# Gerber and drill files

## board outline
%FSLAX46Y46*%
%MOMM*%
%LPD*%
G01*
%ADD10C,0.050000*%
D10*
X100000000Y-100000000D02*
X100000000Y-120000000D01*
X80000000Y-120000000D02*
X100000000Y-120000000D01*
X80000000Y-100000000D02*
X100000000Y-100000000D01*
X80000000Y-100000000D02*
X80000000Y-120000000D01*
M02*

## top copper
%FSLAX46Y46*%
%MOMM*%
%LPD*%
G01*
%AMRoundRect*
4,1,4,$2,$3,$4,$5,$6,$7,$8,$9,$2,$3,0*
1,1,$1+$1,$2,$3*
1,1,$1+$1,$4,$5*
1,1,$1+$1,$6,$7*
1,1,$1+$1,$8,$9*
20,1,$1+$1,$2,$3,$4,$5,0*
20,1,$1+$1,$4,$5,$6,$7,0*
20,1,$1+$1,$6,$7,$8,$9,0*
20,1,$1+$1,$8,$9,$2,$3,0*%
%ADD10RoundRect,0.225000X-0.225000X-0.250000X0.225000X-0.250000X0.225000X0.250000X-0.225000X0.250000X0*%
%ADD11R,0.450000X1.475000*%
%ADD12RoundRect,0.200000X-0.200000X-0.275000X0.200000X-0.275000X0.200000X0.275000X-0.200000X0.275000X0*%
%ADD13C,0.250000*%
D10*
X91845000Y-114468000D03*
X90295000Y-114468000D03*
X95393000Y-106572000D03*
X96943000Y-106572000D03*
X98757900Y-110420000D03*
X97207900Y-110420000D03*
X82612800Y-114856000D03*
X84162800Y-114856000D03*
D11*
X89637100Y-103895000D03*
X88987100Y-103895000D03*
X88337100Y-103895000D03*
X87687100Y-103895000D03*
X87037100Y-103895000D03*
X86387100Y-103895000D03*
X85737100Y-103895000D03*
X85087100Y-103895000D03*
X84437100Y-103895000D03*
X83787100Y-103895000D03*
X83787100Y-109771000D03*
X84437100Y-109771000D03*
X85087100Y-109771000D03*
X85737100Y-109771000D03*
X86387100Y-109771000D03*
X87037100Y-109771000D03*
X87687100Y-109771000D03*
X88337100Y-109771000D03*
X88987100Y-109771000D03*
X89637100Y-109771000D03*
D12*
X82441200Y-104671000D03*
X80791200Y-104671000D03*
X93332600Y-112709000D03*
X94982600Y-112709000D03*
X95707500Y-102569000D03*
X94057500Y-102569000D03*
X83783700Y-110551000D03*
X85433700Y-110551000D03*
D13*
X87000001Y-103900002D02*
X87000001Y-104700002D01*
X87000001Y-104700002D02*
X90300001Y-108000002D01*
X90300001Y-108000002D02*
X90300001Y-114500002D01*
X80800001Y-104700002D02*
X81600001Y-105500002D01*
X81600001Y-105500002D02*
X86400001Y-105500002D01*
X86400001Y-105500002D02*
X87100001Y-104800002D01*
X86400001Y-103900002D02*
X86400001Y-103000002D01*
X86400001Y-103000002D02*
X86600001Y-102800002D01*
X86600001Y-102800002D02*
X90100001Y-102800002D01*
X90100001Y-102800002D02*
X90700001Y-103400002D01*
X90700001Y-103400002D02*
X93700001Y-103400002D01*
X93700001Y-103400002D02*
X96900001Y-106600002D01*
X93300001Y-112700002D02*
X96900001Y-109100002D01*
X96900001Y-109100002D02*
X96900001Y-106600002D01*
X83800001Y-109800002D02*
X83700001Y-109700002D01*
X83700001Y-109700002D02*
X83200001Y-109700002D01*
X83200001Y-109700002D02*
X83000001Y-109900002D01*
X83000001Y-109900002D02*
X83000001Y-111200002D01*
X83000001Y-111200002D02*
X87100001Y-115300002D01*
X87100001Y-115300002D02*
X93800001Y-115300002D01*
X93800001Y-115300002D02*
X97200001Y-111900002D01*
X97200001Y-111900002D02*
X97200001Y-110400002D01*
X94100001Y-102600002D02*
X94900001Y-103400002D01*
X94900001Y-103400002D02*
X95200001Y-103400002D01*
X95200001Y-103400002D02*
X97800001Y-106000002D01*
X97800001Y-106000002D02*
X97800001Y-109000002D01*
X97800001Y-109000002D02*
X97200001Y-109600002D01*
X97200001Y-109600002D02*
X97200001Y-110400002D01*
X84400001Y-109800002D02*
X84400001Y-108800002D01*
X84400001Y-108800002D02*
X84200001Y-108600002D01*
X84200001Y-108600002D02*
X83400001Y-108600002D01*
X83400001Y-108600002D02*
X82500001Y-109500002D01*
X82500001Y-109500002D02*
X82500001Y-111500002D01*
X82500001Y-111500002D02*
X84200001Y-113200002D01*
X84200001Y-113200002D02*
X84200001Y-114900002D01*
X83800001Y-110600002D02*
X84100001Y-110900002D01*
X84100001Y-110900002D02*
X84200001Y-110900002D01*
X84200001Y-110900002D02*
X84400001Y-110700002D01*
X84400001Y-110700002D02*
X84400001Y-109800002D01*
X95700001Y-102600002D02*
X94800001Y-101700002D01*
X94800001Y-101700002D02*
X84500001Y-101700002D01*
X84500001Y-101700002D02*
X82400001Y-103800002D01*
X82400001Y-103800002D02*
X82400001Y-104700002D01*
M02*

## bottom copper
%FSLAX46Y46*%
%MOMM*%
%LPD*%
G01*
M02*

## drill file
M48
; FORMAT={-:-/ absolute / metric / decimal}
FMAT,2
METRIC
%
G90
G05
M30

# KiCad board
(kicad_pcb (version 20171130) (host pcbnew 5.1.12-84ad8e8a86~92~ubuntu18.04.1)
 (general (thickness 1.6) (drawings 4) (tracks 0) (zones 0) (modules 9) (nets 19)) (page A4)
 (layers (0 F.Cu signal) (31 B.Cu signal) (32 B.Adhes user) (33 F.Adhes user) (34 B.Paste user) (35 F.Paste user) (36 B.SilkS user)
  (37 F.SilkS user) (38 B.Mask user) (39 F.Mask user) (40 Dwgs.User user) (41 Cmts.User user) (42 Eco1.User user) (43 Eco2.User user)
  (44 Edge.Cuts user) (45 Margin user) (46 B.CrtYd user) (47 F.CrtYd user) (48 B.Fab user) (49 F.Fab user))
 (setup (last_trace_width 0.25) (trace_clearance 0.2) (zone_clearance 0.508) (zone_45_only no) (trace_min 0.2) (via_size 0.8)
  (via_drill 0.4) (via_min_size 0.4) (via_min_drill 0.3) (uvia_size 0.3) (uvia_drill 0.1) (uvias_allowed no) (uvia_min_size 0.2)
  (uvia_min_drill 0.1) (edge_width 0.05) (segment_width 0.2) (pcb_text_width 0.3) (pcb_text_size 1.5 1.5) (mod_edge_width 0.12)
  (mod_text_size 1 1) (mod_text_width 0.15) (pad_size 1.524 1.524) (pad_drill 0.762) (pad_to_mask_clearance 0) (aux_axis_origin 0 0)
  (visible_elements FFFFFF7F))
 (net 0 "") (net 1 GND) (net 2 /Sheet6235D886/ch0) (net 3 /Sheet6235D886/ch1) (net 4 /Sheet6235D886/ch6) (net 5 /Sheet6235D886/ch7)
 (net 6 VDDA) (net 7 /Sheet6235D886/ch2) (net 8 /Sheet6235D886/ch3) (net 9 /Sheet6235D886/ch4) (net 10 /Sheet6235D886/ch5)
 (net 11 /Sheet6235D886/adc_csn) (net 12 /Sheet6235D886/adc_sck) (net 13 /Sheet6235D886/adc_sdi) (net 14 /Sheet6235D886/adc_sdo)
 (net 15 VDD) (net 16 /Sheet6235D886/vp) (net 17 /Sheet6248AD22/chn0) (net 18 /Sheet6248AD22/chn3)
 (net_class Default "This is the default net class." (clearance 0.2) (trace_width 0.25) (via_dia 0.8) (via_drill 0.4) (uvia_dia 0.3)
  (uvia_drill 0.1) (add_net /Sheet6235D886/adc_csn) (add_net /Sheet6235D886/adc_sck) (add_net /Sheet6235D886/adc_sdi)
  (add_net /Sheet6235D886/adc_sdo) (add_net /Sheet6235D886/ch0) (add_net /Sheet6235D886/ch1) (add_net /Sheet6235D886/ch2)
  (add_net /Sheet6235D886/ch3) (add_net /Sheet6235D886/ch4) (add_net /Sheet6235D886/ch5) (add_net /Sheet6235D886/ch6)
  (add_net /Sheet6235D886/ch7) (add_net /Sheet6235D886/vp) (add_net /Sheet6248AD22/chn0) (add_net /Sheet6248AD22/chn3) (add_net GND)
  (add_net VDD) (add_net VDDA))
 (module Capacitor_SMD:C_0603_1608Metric (layer F.Cu) (at 91.070000 114.468000)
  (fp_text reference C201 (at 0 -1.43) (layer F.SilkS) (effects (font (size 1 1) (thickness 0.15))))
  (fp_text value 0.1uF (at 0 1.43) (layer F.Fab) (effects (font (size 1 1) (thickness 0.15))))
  (pad 2 smd roundrect (at 0.775 0) (size 0.9 0.95) (layers F.Cu F.Mask F.Paste) (roundrect_rratio 0.25) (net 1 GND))
  (pad 1 smd roundrect (at -0.775 0) (size 0.9 0.95) (layers F.Cu F.Mask F.Paste) (roundrect_rratio 0.25) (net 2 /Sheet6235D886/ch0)))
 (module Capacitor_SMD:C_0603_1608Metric (layer F.Cu) (at 96.168000 106.572000)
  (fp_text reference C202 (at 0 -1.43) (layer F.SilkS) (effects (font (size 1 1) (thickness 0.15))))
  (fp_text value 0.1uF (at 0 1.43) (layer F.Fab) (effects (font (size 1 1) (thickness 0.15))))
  (pad 1 smd roundrect (at -0.775 0) (size 0.9 0.95) (layers F.Cu F.Mask F.Paste) (roundrect_rratio 0.25) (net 1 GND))
  (pad 2 smd roundrect (at 0.775 0) (size 0.9 0.95) (layers F.Cu F.Mask F.Paste) (roundrect_rratio 0.25) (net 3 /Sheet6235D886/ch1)))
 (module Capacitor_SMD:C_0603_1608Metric (layer F.Cu) (at 97.982900 110.420000)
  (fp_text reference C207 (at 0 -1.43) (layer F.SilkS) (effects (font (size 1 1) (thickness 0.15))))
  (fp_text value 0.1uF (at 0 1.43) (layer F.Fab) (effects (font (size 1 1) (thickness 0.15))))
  (pad 2 smd roundrect (at 0.775 0) (size 0.9 0.95) (layers F.Cu F.Mask F.Paste) (roundrect_rratio 0.25) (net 1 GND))
  (pad 1 smd roundrect (at -0.775 0) (size 0.9 0.95) (layers F.Cu F.Mask F.Paste) (roundrect_rratio 0.25) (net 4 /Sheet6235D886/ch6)))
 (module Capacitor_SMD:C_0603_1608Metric (layer F.Cu) (at 83.387800 114.856000)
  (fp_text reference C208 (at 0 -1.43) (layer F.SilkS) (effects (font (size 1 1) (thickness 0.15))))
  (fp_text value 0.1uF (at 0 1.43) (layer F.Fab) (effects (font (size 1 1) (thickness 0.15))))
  (pad 1 smd roundrect (at -0.775 0) (size 0.9 0.95) (layers F.Cu F.Mask F.Paste) (roundrect_rratio 0.25) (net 1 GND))
  (pad 2 smd roundrect (at 0.775 0) (size 0.9 0.95) (layers F.Cu F.Mask F.Paste) (roundrect_rratio 0.25) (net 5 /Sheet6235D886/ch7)))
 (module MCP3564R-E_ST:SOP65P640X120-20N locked (layer F.Cu) (at 86.712100 106.833000 270.000000)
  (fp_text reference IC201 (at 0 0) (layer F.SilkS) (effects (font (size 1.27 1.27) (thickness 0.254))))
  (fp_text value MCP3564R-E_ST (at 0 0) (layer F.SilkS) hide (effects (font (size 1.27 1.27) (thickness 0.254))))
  (pad 1 smd rect (at -2.938 -2.925) (size 0.45 1.475) (layers F.Cu F.Mask F.Paste) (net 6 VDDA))
  (pad 2 smd rect (at -2.938 -2.275) (size 0.45 1.475) (layers F.Cu F.Mask F.Paste) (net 1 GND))
  (pad 3 smd rect (at -2.938 -1.625) (size 0.45 1.475) (layers F.Cu F.Mask F.Paste) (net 1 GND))
  (pad 4 smd rect (at -2.938 -0.975) (size 0.45 1.475) (layers F.Cu F.Mask F.Paste))
  (pad 5 smd rect (at -2.938 -0.325) (size 0.45 1.475) (layers F.Cu F.Mask F.Paste) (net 2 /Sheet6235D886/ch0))
  (pad 6 smd rect (at -2.938 0.325) (size 0.45 1.475) (layers F.Cu F.Mask F.Paste) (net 3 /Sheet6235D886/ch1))
  (pad 7 smd rect (at -2.938 0.975) (size 0.45 1.475) (layers F.Cu F.Mask F.Paste) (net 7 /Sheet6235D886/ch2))
  (pad 8 smd rect (at -2.938 1.625) (size 0.45 1.475) (layers F.Cu F.Mask F.Paste) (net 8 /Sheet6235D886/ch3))
  (pad 9 smd rect (at -2.938 2.275) (size 0.45 1.475) (layers F.Cu F.Mask F.Paste) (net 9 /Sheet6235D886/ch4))
  (pad 10 smd rect (at -2.938 2.925) (size 0.45 1.475) (layers F.Cu F.Mask F.Paste) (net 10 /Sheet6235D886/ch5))
  (pad 11 smd rect (at 2.938 2.925) (size 0.45 1.475) (layers F.Cu F.Mask F.Paste) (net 4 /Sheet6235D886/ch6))
  (pad 12 smd rect (at 2.938 2.275) (size 0.45 1.475) (layers F.Cu F.Mask F.Paste) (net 5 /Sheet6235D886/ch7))
  (pad 13 smd rect (at 2.938 1.625) (size 0.45 1.475) (layers F.Cu F.Mask F.Paste) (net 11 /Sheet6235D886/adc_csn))
  (pad 14 smd rect (at 2.938 0.975) (size 0.45 1.475) (layers F.Cu F.Mask F.Paste) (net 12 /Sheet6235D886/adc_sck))
  (pad 15 smd rect (at 2.938 0.325) (size 0.45 1.475) (layers F.Cu F.Mask F.Paste) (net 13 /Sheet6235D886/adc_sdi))
  (pad 16 smd rect (at 2.938 -0.325) (size 0.45 1.475) (layers F.Cu F.Mask F.Paste) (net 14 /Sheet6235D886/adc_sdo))
  (pad 17 smd rect (at 2.938 -0.975) (size 0.45 1.475) (layers F.Cu F.Mask F.Paste))
  (pad 18 smd rect (at 2.938 -1.625) (size 0.45 1.475) (layers F.Cu F.Mask F.Paste))
  (pad 19 smd rect (at 2.938 -2.275) (size 0.45 1.475) (layers F.Cu F.Mask F.Paste) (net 1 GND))
  (pad 20 smd rect (at 2.938 -2.925) (size 0.45 1.475) (layers F.Cu F.Mask F.Paste) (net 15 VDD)))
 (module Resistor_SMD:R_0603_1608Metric (layer F.Cu) (at 81.616200 104.671000)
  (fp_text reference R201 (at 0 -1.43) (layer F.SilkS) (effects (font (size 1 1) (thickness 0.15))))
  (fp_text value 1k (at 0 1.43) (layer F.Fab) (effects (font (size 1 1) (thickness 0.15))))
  (pad 2 smd roundrect (at 0.825 0) (size 0.8 0.95) (layers F.Cu F.Mask F.Paste) (roundrect_rratio 0.25) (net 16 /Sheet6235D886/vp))
  (pad 1 smd roundrect (at -0.825 0) (size 0.8 0.95) (layers F.Cu F.Mask F.Paste) (roundrect_rratio 0.25) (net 2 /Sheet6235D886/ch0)))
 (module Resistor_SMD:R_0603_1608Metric (layer F.Cu) (at 94.157600 112.709000)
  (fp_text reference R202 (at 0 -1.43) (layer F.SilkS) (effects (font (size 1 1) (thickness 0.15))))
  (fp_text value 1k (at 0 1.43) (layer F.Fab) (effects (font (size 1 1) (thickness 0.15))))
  (pad 1 smd roundrect (at -0.825 0) (size 0.8 0.95) (layers F.Cu F.Mask F.Paste) (roundrect_rratio 0.25) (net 3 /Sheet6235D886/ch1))
  (pad 2 smd roundrect (at 0.825 0) (size 0.8 0.95) (layers F.Cu F.Mask F.Paste) (roundrect_rratio 0.25) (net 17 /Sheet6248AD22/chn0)))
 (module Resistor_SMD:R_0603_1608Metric (layer F.Cu) (at 94.882500 102.569000)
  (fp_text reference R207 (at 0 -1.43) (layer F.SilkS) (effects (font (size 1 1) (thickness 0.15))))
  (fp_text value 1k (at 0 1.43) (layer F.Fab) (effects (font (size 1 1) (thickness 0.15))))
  (pad 2 smd roundrect (at 0.825 0) (size 0.8 0.95) (layers F.Cu F.Mask F.Paste) (roundrect_rratio 0.25) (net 16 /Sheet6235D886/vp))
  (pad 1 smd roundrect (at -0.825 0) (size 0.8 0.95) (layers F.Cu F.Mask F.Paste) (roundrect_rratio 0.25) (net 4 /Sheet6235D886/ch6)))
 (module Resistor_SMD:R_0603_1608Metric (layer F.Cu) (at 84.608700 110.551000)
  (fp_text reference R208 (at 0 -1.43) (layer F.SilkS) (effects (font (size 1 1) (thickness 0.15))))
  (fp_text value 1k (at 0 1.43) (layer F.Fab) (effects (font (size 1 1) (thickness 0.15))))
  (pad 1 smd roundrect (at -0.825 0) (size 0.8 0.95) (layers F.Cu F.Mask F.Paste) (roundrect_rratio 0.25) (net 5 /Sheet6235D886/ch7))
  (pad 2 smd roundrect (at 0.825 0) (size 0.8 0.95) (layers F.Cu F.Mask F.Paste) (roundrect_rratio 0.25) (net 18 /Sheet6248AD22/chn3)))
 (gr_line (start 100 100) (end 100 120) (layer Edge.Cuts) (width 0.05))
 (gr_line (start 80 120) (end 100 120) (layer Edge.Cuts) (width 0.05))
 (gr_line (start 80 100) (end 100 100) (layer Edge.Cuts) (width 0.05))
 (gr_line (start 80 100) (end 80 120) (layer Edge.Cuts) (width 0.05))
 (segment (start 87.000001 103.900002) (end 87.000001 104.700002) (width 0.250000) (layer F.Cu) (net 2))
 (segment (start 87.000001 104.700002) (end 90.300001 108.000002) (width 0.250000) (layer F.Cu) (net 2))
 (segment (start 90.300001 108.000002) (end 90.300001 114.500002) (width 0.250000) (layer F.Cu) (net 2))
 (segment (start 80.800001 104.700002) (end 81.600001 105.500002) (width 0.250000) (layer F.Cu) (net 2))
 (segment (start 81.600001 105.500002) (end 86.400001 105.500002) (width 0.250000) (layer F.Cu) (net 2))
 (segment (start 86.400001 105.500002) (end 87.100001 104.800002) (width 0.250000) (layer F.Cu) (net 2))
 (segment (start 86.400001 103.900002) (end 86.400001 103.000002) (width 0.250000) (layer F.Cu) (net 3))
 (segment (start 86.400001 103.000002) (end 86.600001 102.800002) (width 0.250000) (layer F.Cu) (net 3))
 (segment (start 86.600001 102.800002) (end 90.100001 102.800002) (width 0.250000) (layer F.Cu) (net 3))
 (segment (start 90.100001 102.800002) (end 90.700001 103.400002) (width 0.250000) (layer F.Cu) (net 3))
 (segment (start 90.700001 103.400002) (end 93.700001 103.400002) (width 0.250000) (layer F.Cu) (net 3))
 (segment (start 93.700001 103.400002) (end 96.900001 106.600002) (width 0.250000) (layer F.Cu) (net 3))
 (segment (start 93.300001 112.700002) (end 96.900001 109.100002) (width 0.250000) (layer F.Cu) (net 3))
 (segment (start 96.900001 109.100002) (end 96.900001 106.600002) (width 0.250000) (layer F.Cu) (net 3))
 (segment (start 83.800001 109.800002) (end 83.700001 109.700002) (width 0.250000) (layer F.Cu) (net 4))
 (segment (start 83.700001 109.700002) (end 83.200001 109.700002) (width 0.250000) (layer F.Cu) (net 4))
 (segment (start 83.200001 109.700002) (end 83.000001 109.900002) (width 0.250000) (layer F.Cu) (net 4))
 (segment (start 83.000001 109.900002) (end 83.000001 111.200002) (width 0.250000) (layer F.Cu) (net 4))
 (segment (start 83.000001 111.200002) (end 87.100001 115.300002) (width 0.250000) (layer F.Cu) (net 4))
 (segment (start 87.100001 115.300002) (end 93.800001 115.300002) (width 0.250000) (layer F.Cu) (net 4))
 (segment (start 93.800001 115.300002) (end 97.200001 111.900002) (width 0.250000) (layer F.Cu) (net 4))
 (segment (start 97.200001 111.900002) (end 97.200001 110.400002) (width 0.250000) (layer F.Cu) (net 4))
 (segment (start 94.100001 102.600002) (end 94.900001 103.400002) (width 0.250000) (layer F.Cu) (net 4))
 (segment (start 94.900001 103.400002) (end 95.200001 103.400002) (width 0.250000) (layer F.Cu) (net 4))
 (segment (start 95.200001 103.400002) (end 97.800001 106.000002) (width 0.250000) (layer F.Cu) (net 4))
 (segment (start 97.800001 106.000002) (end 97.800001 109.000002) (width 0.250000) (layer F.Cu) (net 4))
 (segment (start 97.800001 109.000002) (end 97.200001 109.600002) (width 0.250000) (layer F.Cu) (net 4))
 (segment (start 97.200001 109.600002) (end 97.200001 110.400002) (width 0.250000) (layer F.Cu) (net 4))
 (segment (start 84.400001 109.800002) (end 84.400001 108.800002) (width 0.250000) (layer F.Cu) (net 5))
 (segment (start 84.400001 108.800002) (end 84.200001 108.600002) (width 0.250000) (layer F.Cu) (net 5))
 (segment (start 84.200001 108.600002) (end 83.400001 108.600002) (width 0.250000) (layer F.Cu) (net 5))
 (segment (start 83.400001 108.600002) (end 82.500001 109.500002) (width 0.250000) (layer F.Cu) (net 5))
 (segment (start 82.500001 109.500002) (end 82.500001 111.500002) (width 0.250000) (layer F.Cu) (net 5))
 (segment (start 82.500001 111.500002) (end 84.200001 113.200002) (width 0.250000) (layer F.Cu) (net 5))
 (segment (start 84.200001 113.200002) (end 84.200001 114.900002) (width 0.250000) (layer F.Cu) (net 5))
 (segment (start 83.800001 110.600002) (end 84.100001 110.900002) (width 0.250000) (layer F.Cu) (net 5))
 (segment (start 84.100001 110.900002) (end 84.200001 110.900002) (width 0.250000) (layer F.Cu) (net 5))
 (segment (start 84.200001 110.900002) (end 84.400001 110.700002) (width 0.250000) (layer F.Cu) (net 5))
 (segment (start 84.400001 110.700002) (end 84.400001 109.800002) (width 0.250000) (layer F.Cu) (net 5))
 (segment (start 95.700001 102.600002) (end 94.800001 101.700002) (width 0.250000) (layer F.Cu) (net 16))
 (segment (start 94.800001 101.700002) (end 84.500001 101.700002) (width 0.250000) (layer F.Cu) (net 16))
 (segment (start 84.500001 101.700002) (end 82.400001 103.800002) (width 0.250000) (layer F.Cu) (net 16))
 (segment (start 82.400001 103.800002) (end 82.400001 104.700002) (width 0.250000) (layer F.Cu) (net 16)))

